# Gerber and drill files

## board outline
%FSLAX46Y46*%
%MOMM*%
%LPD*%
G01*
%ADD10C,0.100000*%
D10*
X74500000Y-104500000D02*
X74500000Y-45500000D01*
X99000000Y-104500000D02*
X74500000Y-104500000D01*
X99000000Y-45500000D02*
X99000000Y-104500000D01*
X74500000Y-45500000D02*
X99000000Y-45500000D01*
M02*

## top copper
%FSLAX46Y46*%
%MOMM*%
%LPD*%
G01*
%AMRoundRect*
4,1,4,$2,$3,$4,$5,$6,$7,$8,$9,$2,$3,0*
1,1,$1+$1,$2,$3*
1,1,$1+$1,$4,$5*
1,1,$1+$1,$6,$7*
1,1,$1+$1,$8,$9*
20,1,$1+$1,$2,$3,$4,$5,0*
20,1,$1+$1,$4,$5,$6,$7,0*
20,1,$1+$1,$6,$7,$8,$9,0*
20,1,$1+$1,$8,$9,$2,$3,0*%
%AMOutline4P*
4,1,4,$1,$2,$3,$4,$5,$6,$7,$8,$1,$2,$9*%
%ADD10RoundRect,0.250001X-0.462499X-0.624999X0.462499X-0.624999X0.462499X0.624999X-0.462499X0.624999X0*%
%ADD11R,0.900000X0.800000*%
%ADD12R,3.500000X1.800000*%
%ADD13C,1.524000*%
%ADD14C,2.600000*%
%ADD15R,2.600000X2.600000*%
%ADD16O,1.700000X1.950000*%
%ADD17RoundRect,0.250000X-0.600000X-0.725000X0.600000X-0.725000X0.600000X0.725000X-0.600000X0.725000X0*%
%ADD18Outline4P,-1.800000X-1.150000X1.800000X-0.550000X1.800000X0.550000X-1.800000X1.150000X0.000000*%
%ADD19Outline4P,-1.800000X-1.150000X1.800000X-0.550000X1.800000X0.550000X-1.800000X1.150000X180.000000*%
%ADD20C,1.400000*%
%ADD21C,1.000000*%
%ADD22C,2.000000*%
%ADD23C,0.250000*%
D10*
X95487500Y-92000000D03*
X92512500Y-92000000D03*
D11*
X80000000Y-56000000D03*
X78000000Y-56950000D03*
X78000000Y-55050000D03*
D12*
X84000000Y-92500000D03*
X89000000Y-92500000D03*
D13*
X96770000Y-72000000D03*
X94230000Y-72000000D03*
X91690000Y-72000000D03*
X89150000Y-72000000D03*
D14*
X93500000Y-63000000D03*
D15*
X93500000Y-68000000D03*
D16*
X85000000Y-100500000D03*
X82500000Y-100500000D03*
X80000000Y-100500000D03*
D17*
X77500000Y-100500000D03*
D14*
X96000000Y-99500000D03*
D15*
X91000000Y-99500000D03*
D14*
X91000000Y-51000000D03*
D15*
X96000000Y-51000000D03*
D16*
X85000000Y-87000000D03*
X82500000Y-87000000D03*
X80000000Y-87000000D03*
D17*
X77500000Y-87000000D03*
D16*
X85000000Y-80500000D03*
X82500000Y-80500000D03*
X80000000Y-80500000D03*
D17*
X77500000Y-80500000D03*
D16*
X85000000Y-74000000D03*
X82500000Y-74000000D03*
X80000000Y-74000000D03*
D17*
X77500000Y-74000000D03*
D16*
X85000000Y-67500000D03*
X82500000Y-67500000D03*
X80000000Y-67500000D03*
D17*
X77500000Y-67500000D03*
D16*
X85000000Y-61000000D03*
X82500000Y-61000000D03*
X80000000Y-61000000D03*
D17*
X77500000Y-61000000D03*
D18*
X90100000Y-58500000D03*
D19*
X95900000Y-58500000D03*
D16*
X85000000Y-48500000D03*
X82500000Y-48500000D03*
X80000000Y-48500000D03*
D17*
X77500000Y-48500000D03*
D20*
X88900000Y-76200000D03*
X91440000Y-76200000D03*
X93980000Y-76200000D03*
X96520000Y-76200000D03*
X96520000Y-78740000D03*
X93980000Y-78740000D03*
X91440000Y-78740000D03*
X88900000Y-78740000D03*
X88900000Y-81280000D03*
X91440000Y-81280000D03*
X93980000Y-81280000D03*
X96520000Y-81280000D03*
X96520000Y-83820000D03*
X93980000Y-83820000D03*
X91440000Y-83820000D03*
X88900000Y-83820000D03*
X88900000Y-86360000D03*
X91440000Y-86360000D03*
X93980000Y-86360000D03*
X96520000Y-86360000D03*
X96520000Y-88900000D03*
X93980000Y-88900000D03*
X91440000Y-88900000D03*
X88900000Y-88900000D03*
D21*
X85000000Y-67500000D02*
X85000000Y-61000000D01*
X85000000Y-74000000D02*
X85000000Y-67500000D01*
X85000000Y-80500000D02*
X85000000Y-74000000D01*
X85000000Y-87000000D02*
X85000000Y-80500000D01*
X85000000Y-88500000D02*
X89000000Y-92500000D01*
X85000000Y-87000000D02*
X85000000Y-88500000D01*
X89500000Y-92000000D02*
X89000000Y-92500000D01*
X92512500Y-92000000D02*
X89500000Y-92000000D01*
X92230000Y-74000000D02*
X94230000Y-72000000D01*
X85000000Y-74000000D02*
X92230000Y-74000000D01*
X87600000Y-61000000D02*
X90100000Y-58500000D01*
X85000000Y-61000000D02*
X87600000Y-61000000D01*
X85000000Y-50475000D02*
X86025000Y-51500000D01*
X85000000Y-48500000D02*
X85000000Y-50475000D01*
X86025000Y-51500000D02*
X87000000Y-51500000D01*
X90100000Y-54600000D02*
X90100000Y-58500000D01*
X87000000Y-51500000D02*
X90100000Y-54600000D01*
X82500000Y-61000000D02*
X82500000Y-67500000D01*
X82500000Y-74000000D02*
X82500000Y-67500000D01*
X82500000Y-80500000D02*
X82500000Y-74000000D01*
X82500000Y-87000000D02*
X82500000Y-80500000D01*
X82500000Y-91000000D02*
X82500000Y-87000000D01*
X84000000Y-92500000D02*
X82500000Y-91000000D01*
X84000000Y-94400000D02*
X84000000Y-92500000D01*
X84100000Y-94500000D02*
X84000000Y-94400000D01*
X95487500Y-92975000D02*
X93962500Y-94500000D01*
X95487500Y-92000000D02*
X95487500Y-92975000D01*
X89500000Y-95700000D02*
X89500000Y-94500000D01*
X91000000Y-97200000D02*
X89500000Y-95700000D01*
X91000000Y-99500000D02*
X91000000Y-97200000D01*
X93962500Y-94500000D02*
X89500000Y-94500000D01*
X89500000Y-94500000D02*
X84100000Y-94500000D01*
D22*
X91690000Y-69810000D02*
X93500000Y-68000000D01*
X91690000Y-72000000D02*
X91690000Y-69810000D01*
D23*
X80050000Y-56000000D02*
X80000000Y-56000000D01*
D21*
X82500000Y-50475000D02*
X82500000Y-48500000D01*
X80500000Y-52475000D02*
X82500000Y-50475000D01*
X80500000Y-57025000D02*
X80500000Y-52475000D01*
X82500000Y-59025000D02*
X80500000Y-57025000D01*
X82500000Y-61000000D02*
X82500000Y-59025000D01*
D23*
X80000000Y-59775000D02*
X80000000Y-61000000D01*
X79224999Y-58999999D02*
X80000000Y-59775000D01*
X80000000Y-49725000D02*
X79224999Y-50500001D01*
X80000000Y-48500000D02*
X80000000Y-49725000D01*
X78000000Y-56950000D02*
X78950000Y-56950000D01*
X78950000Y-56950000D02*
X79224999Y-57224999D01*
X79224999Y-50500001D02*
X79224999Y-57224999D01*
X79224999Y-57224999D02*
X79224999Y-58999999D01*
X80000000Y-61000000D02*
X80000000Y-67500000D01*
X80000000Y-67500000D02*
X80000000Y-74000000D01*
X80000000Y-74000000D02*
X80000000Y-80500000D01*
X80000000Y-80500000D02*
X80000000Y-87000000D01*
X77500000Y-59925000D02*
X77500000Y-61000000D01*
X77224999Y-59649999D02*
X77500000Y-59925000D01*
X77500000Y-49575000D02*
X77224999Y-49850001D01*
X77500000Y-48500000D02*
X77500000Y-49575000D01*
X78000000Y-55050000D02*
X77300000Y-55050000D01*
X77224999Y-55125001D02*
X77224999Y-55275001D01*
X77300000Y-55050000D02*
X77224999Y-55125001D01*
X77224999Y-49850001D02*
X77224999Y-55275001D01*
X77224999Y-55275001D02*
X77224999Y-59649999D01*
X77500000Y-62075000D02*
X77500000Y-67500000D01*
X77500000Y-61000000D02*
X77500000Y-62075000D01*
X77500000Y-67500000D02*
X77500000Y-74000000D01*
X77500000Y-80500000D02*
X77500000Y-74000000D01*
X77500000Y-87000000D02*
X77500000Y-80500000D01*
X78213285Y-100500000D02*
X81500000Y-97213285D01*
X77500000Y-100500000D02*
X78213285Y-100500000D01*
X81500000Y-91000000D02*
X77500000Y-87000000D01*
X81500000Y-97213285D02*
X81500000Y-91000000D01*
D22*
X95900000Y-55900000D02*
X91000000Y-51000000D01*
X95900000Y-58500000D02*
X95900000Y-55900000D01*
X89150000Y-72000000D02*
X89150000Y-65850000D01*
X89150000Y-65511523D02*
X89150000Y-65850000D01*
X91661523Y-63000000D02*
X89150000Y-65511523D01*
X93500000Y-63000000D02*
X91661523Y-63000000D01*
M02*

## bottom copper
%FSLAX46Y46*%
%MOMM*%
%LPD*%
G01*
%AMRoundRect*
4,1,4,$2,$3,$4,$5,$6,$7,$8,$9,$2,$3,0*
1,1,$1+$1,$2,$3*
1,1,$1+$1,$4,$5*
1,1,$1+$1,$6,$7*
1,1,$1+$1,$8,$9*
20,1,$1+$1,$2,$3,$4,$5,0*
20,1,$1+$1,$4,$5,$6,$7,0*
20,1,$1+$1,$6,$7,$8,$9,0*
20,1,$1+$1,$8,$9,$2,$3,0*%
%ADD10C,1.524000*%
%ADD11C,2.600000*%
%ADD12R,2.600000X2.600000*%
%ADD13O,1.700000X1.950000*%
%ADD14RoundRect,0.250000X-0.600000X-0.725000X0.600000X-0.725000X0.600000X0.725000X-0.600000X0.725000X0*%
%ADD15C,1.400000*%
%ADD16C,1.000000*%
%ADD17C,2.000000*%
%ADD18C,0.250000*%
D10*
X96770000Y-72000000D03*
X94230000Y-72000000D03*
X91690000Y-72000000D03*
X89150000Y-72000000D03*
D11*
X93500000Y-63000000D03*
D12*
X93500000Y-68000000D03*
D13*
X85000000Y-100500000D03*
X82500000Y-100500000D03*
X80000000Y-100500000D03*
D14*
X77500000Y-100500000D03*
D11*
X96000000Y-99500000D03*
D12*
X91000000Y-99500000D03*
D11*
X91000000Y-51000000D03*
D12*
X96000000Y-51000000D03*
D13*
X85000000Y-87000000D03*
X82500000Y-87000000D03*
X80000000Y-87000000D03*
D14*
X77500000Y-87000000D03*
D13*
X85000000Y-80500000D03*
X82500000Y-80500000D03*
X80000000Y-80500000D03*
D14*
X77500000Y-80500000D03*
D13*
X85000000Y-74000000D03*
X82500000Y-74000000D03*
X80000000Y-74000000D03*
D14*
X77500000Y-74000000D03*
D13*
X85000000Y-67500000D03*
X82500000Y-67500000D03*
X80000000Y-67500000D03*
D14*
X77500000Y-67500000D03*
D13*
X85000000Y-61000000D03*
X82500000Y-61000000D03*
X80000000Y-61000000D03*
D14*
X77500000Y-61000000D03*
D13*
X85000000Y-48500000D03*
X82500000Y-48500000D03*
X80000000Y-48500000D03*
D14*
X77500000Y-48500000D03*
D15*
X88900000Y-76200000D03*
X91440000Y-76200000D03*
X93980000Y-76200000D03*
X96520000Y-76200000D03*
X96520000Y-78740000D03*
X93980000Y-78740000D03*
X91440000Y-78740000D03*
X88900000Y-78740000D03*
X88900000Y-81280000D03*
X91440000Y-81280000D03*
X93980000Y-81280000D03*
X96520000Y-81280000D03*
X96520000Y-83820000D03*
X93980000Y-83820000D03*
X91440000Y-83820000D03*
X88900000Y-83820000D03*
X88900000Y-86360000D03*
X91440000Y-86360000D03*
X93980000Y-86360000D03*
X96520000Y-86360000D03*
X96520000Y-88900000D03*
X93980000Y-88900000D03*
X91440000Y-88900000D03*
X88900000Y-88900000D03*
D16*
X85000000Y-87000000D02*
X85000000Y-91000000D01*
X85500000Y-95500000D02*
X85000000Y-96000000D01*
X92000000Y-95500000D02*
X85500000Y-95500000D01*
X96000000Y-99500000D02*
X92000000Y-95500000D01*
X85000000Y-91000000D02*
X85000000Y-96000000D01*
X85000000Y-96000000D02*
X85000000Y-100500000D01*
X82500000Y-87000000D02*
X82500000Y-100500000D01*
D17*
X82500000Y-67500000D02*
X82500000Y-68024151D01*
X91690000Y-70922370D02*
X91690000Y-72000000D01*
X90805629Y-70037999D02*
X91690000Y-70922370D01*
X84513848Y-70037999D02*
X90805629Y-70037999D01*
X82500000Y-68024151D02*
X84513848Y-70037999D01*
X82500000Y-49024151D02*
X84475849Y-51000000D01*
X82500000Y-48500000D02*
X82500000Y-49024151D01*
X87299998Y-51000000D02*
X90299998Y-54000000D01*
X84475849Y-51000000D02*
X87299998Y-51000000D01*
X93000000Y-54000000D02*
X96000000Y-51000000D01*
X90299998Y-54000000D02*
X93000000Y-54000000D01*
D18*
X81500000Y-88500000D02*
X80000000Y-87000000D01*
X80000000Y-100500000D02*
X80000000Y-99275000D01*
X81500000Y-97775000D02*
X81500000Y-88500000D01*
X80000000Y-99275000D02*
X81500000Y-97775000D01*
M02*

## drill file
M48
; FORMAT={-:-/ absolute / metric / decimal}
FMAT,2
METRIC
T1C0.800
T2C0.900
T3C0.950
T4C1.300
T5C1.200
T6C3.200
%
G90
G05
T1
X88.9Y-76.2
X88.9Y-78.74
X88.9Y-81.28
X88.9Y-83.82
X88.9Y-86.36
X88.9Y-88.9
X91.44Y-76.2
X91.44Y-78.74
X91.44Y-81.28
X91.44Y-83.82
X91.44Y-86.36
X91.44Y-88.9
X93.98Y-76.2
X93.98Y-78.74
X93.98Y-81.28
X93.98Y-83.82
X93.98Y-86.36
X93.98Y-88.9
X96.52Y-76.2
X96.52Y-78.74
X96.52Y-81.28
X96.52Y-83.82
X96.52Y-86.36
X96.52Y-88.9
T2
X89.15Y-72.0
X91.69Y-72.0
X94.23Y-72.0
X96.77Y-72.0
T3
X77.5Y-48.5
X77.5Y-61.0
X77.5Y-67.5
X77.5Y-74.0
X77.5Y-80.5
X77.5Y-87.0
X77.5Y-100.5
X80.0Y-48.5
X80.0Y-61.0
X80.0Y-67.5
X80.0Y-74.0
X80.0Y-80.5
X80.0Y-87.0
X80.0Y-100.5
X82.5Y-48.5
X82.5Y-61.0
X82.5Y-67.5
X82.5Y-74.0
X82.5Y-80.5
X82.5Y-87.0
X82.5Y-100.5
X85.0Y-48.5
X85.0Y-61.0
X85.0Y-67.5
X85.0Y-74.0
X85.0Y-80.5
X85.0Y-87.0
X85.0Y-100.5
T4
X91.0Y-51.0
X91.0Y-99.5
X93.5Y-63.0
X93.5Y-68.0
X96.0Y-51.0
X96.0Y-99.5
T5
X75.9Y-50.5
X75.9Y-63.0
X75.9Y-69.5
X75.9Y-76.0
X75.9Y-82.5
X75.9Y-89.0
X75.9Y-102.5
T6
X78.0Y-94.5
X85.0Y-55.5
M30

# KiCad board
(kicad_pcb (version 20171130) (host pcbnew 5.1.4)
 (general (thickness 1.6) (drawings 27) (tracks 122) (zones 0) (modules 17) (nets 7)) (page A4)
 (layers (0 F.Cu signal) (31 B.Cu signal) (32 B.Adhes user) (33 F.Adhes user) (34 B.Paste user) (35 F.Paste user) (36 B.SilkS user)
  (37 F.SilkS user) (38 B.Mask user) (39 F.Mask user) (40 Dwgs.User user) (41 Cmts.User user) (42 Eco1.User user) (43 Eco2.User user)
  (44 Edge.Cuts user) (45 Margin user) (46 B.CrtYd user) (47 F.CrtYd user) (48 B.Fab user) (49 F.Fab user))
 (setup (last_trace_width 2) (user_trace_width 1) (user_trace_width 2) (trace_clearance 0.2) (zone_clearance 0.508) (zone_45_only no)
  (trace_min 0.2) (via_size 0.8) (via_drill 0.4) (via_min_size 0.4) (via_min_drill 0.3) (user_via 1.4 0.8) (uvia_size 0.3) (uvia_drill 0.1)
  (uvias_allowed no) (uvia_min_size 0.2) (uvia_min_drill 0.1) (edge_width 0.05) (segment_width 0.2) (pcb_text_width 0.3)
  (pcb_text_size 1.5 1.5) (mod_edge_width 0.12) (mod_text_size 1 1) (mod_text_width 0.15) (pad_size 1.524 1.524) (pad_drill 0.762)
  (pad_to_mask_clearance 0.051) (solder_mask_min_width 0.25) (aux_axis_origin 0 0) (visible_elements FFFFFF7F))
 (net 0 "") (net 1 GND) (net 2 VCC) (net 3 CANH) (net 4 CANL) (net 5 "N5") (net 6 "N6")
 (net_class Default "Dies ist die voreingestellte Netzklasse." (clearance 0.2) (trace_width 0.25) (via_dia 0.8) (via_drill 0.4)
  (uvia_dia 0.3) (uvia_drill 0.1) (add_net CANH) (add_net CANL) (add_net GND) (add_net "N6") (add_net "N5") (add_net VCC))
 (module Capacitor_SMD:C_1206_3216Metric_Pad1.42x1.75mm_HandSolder (layer F.Cu) (at 94 92)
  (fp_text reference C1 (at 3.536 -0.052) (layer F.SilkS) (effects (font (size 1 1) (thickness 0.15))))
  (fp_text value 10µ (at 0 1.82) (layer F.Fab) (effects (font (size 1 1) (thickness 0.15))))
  (pad 2 smd roundrect (at 1.4875 0) (size 1.425 1.75) (layers F.Cu F.Paste F.Mask) (roundrect_rratio 0.175439) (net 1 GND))
  (pad 1 smd roundrect (at -1.4875 0) (size 1.425 1.75) (layers F.Cu F.Paste F.Mask) (roundrect_rratio 0.175439) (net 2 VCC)))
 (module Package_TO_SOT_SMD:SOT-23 (layer F.Cu) (at 79 56)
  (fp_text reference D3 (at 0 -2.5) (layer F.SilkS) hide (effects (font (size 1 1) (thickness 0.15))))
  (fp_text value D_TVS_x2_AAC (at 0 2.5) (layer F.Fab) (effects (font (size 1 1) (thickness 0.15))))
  (pad 3 smd rect (at 1 0) (size 0.9 0.8) (layers F.Cu F.Paste F.Mask) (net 1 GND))
  (pad 2 smd rect (at -1 0.95) (size 0.9 0.8) (layers F.Cu F.Paste F.Mask) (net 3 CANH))
  (pad 1 smd rect (at -1 -0.95) (size 0.9 0.8) (layers F.Cu F.Paste F.Mask) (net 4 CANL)))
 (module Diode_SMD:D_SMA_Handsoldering (layer F.Cu) (at 86.5 92.5 180)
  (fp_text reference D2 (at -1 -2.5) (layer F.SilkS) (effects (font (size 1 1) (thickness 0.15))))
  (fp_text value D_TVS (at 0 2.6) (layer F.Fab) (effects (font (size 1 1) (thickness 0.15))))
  (pad 2 smd rect (at 2.5 0 180) (size 3.5 1.8) (layers F.Cu F.Paste F.Mask) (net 1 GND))
  (pad 1 smd rect (at -2.5 0 180) (size 3.5 1.8) (layers F.Cu F.Paste F.Mask) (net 2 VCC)))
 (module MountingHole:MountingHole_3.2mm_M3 (layer F.Cu) (at 78 94.5)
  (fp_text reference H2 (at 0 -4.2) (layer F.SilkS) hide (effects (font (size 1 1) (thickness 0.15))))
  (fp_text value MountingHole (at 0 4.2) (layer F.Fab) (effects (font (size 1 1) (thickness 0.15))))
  (pad 1 np_thru_hole circle (at 0 0) (size 3.2 3.2) (drill 3.2) (layers *.Cu *.Mask)))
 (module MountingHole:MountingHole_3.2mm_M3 (layer F.Cu) (at 85 55.5)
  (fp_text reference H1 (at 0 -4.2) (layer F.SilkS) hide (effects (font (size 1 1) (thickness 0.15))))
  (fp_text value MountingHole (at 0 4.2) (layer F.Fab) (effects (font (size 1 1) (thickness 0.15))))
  (pad 1 np_thru_hole circle (at 0 0) (size 3.2 3.2) (drill 3.2) (layers *.Cu *.Mask)))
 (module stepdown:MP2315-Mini (layer F.Cu) (at 93 81)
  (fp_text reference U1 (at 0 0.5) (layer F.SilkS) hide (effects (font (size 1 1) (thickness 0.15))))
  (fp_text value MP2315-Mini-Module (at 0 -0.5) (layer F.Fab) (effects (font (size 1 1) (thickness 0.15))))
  (pad 4 thru_hole circle (at 3.77 -9) (size 1.524 1.524) (drill 0.9) (layers *.Cu *.Mask))
  (pad 3 thru_hole circle (at 1.23 -9) (size 1.524 1.524) (drill 0.9) (layers *.Cu *.Mask) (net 2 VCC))
  (pad 2 thru_hole circle (at -1.31 -9) (size 1.524 1.524) (drill 0.9) (layers *.Cu *.Mask) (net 1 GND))
  (pad 1 thru_hole circle (at -3.85 -9) (size 1.524 1.524) (drill 0.9) (layers *.Cu *.Mask) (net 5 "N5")))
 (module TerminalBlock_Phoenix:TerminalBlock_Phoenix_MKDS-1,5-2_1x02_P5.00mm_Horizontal (layer F.Cu) (at 93.5 68 90)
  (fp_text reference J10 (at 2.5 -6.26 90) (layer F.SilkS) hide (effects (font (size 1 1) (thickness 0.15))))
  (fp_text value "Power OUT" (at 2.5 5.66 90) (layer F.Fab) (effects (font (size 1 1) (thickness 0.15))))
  (pad 2 thru_hole circle (at 5 0 90) (size 2.6 2.6) (drill 1.3) (layers *.Cu *.Mask) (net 5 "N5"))
  (pad 1 thru_hole rect (at 0 0 90) (size 2.6 2.6) (drill 1.3) (layers *.Cu *.Mask) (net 1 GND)))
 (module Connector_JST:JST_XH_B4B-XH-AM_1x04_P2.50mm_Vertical (layer F.Cu) (at 77.5 100.5)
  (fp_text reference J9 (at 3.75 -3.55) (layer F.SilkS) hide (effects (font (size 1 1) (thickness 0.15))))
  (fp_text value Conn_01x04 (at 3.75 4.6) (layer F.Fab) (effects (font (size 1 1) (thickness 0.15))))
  (pad "" np_thru_hole circle (at -1.6 2) (size 1.2 1.2) (drill 1.2) (layers *.Cu *.Mask))
  (pad 4 thru_hole oval (at 7.5 0) (size 1.7 1.95) (drill 0.95) (layers *.Cu *.Mask) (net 2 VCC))
  (pad 3 thru_hole oval (at 5 0) (size 1.7 1.95) (drill 0.95) (layers *.Cu *.Mask) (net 1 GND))
  (pad 2 thru_hole oval (at 2.5 0) (size 1.7 1.95) (drill 0.95) (layers *.Cu *.Mask) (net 3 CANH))
  (pad 1 thru_hole roundrect (at 0 0) (size 1.7 1.95) (drill 0.95) (layers *.Cu *.Mask) (roundrect_rratio 0.147059) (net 4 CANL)))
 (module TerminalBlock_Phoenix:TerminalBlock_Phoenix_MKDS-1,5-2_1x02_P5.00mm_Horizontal (layer F.Cu) (at 91 99.5)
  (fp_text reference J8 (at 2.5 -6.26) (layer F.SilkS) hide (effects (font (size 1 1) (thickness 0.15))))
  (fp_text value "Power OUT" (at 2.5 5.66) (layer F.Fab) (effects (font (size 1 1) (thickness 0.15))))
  (pad 2 thru_hole circle (at 5 0) (size 2.6 2.6) (drill 1.3) (layers *.Cu *.Mask) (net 2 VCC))
  (pad 1 thru_hole rect (at 0 0) (size 2.6 2.6) (drill 1.3) (layers *.Cu *.Mask) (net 1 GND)))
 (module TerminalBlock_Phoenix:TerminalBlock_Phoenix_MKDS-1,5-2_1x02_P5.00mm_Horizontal (layer F.Cu) (at 96 51 180)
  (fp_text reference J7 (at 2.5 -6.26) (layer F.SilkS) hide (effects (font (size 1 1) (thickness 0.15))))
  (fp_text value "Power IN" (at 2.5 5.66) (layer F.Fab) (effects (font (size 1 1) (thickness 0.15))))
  (pad 2 thru_hole circle (at 5 0 180) (size 2.6 2.6) (drill 1.3) (layers *.Cu *.Mask) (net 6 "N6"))
  (pad 1 thru_hole rect (at 0 0 180) (size 2.6 2.6) (drill 1.3) (layers *.Cu *.Mask) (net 1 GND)))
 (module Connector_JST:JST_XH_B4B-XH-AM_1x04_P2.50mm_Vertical (layer F.Cu) (at 77.5 87)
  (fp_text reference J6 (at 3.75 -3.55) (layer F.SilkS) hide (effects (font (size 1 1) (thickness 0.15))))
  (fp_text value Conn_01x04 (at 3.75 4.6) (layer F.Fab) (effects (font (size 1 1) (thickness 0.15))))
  (pad "" np_thru_hole circle (at -1.6 2) (size 1.2 1.2) (drill 1.2) (layers *.Cu *.Mask))
  (pad 4 thru_hole oval (at 7.5 0) (size 1.7 1.95) (drill 0.95) (layers *.Cu *.Mask) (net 2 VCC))
  (pad 3 thru_hole oval (at 5 0) (size 1.7 1.95) (drill 0.95) (layers *.Cu *.Mask) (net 1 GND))
  (pad 2 thru_hole oval (at 2.5 0) (size 1.7 1.95) (drill 0.95) (layers *.Cu *.Mask) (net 3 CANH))
  (pad 1 thru_hole roundrect (at 0 0) (size 1.7 1.95) (drill 0.95) (layers *.Cu *.Mask) (roundrect_rratio 0.147059) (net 4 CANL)))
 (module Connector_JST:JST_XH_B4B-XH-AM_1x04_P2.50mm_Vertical (layer F.Cu) (at 77.5 80.5)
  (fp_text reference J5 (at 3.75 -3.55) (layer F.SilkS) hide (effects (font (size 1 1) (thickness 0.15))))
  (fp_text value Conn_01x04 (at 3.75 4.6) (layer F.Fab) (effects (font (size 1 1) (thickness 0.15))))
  (pad "" np_thru_hole circle (at -1.6 2) (size 1.2 1.2) (drill 1.2) (layers *.Cu *.Mask))
  (pad 4 thru_hole oval (at 7.5 0) (size 1.7 1.95) (drill 0.95) (layers *.Cu *.Mask) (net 2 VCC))
  (pad 3 thru_hole oval (at 5 0) (size 1.7 1.95) (drill 0.95) (layers *.Cu *.Mask) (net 1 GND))
  (pad 2 thru_hole oval (at 2.5 0) (size 1.7 1.95) (drill 0.95) (layers *.Cu *.Mask) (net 3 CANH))
  (pad 1 thru_hole roundrect (at 0 0) (size 1.7 1.95) (drill 0.95) (layers *.Cu *.Mask) (roundrect_rratio 0.147059) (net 4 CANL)))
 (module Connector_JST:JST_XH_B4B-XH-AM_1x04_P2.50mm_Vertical (layer F.Cu) (at 77.5 74)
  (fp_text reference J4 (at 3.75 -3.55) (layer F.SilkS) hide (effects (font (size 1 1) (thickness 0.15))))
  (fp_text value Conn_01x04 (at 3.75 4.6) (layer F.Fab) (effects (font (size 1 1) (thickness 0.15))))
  (pad "" np_thru_hole circle (at -1.6 2) (size 1.2 1.2) (drill 1.2) (layers *.Cu *.Mask))
  (pad 4 thru_hole oval (at 7.5 0) (size 1.7 1.95) (drill 0.95) (layers *.Cu *.Mask) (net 2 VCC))
  (pad 3 thru_hole oval (at 5 0) (size 1.7 1.95) (drill 0.95) (layers *.Cu *.Mask) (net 1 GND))
  (pad 2 thru_hole oval (at 2.5 0) (size 1.7 1.95) (drill 0.95) (layers *.Cu *.Mask) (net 3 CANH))
  (pad 1 thru_hole roundrect (at 0 0) (size 1.7 1.95) (drill 0.95) (layers *.Cu *.Mask) (roundrect_rratio 0.147059) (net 4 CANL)))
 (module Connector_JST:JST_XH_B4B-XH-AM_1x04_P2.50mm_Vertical (layer F.Cu) (at 77.5 67.5)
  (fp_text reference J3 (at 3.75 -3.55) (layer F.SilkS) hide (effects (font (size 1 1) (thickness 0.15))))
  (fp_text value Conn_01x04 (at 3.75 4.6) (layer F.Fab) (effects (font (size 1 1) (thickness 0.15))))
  (pad "" np_thru_hole circle (at -1.6 2) (size 1.2 1.2) (drill 1.2) (layers *.Cu *.Mask))
  (pad 4 thru_hole oval (at 7.5 0) (size 1.7 1.95) (drill 0.95) (layers *.Cu *.Mask) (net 2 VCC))
  (pad 3 thru_hole oval (at 5 0) (size 1.7 1.95) (drill 0.95) (layers *.Cu *.Mask) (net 1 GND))
  (pad 2 thru_hole oval (at 2.5 0) (size 1.7 1.95) (drill 0.95) (layers *.Cu *.Mask) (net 3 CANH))
  (pad 1 thru_hole roundrect (at 0 0) (size 1.7 1.95) (drill 0.95) (layers *.Cu *.Mask) (roundrect_rratio 0.147059) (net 4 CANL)))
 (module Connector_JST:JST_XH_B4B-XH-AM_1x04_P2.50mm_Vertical (layer F.Cu) (at 77.5 61)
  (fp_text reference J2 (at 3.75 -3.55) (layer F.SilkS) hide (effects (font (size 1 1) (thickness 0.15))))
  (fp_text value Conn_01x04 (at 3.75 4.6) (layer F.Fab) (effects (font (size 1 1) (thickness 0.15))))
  (pad "" np_thru_hole circle (at -1.6 2) (size 1.2 1.2) (drill 1.2) (layers *.Cu *.Mask))
  (pad 4 thru_hole oval (at 7.5 0) (size 1.7 1.95) (drill 0.95) (layers *.Cu *.Mask) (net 2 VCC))
  (pad 3 thru_hole oval (at 5 0) (size 1.7 1.95) (drill 0.95) (layers *.Cu *.Mask) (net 1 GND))
  (pad 2 thru_hole oval (at 2.5 0) (size 1.7 1.95) (drill 0.95) (layers *.Cu *.Mask) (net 3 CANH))
  (pad 1 thru_hole roundrect (at 0 0) (size 1.7 1.95) (drill 0.95) (layers *.Cu *.Mask) (roundrect_rratio 0.147059) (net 4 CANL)))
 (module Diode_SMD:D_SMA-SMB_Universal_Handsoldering (layer F.Cu) (at 93 58.5 180)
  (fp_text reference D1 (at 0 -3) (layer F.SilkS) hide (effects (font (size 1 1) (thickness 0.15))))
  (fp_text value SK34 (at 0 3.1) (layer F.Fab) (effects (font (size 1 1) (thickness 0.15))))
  (pad 2 smd trapezoid (at 2.9 0) (size 3.6 1.7) (rect_delta 0.6 0) (layers F.Cu F.Paste F.Mask) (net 2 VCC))
  (pad 1 smd trapezoid (at -2.9 0 180) (size 3.6 1.7) (rect_delta 0.6 0) (layers F.Cu F.Paste F.Mask) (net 6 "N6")))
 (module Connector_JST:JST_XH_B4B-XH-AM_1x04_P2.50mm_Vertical (layer F.Cu) (at 77.5 48.5)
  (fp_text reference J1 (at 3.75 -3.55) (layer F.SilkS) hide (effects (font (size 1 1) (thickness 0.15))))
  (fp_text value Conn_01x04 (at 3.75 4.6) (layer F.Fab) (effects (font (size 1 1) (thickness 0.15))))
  (pad "" np_thru_hole circle (at -1.6 2) (size 1.2 1.2) (drill 1.2) (layers *.Cu *.Mask))
  (pad 4 thru_hole oval (at 7.5 0) (size 1.7 1.95) (drill 0.95) (layers *.Cu *.Mask) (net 2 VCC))
  (pad 3 thru_hole oval (at 5 0) (size 1.7 1.95) (drill 0.95) (layers *.Cu *.Mask) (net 1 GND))
  (pad 2 thru_hole oval (at 2.5 0) (size 1.7 1.95) (drill 0.95) (layers *.Cu *.Mask) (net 3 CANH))
  (pad 1 thru_hole roundrect (at 0 0) (size 1.7 1.95) (drill 0.95) (layers *.Cu *.Mask) (roundrect_rratio 0.147059) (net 4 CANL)))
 (gr_line (start 74.5 104.5) (end 74.5 45.5) (layer Edge.Cuts) (width 0.1))
 (gr_line (start 99 104.5) (end 74.5 104.5) (layer Edge.Cuts) (width 0.1))
 (gr_line (start 99 45.5) (end 99 104.5) (layer Edge.Cuts) (width 0.1))
 (gr_line (start 74.5 45.5) (end 99 45.5) (layer Edge.Cuts) (width 0.1))
 (via (at 88.9 76.2) (size 1.4) (drill 0.8) (layers F.Cu B.Cu) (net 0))
 (via (at 91.44 76.2) (size 1.4) (drill 0.8) (layers F.Cu B.Cu) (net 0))
 (via (at 93.98 76.2) (size 1.4) (drill 0.8) (layers F.Cu B.Cu) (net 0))
 (via (at 96.52 76.2) (size 1.4) (drill 0.8) (layers F.Cu B.Cu) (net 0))
 (via (at 96.52 78.74) (size 1.4) (drill 0.8) (layers F.Cu B.Cu) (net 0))
 (via (at 93.98 78.74) (size 1.4) (drill 0.8) (layers F.Cu B.Cu) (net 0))
 (via (at 91.44 78.74) (size 1.4) (drill 0.8) (layers F.Cu B.Cu) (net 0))
 (via (at 88.9 78.74) (size 1.4) (drill 0.8) (layers F.Cu B.Cu) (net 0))
 (via (at 88.9 81.28) (size 1.4) (drill 0.8) (layers F.Cu B.Cu) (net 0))
 (via (at 91.44 81.28) (size 1.4) (drill 0.8) (layers F.Cu B.Cu) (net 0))
 (via (at 93.98 81.28) (size 1.4) (drill 0.8) (layers F.Cu B.Cu) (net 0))
 (via (at 96.52 81.28) (size 1.4) (drill 0.8) (layers F.Cu B.Cu) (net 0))
 (via (at 96.52 83.82) (size 1.4) (drill 0.8) (layers F.Cu B.Cu) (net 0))
 (via (at 93.98 83.82) (size 1.4) (drill 0.8) (layers F.Cu B.Cu) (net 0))
 (via (at 91.44 83.82) (size 1.4) (drill 0.8) (layers F.Cu B.Cu) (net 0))
 (via (at 88.9 83.82) (size 1.4) (drill 0.8) (layers F.Cu B.Cu) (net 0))
 (via (at 88.9 86.36) (size 1.4) (drill 0.8) (layers F.Cu B.Cu) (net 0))
 (via (at 91.44 86.36) (size 1.4) (drill 0.8) (layers F.Cu B.Cu) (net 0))
 (via (at 93.98 86.36) (size 1.4) (drill 0.8) (layers F.Cu B.Cu) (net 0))
 (via (at 96.52 86.36) (size 1.4) (drill 0.8) (layers F.Cu B.Cu) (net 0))
 (via (at 96.52 88.9) (size 1.4) (drill 0.8) (layers F.Cu B.Cu) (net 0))
 (via (at 93.98 88.9) (size 1.4) (drill 0.8) (layers F.Cu B.Cu) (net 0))
 (via (at 91.44 88.9) (size 1.4) (drill 0.8) (layers F.Cu B.Cu) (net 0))
 (via (at 88.9 88.9) (size 1.4) (drill 0.8) (layers F.Cu B.Cu) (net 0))
 (segment (start 85 67.5) (end 85 61) (width 1) (layer F.Cu) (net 2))
 (segment (start 85 74) (end 85 67.5) (width 1) (layer F.Cu) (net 2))
 (segment (start 85 80.5) (end 85 74) (width 1) (layer F.Cu) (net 2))
 (segment (start 85 87) (end 85 80.5) (width 1) (layer F.Cu) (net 2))
 (segment (start 85 88.5) (end 89 92.5) (width 1) (layer F.Cu) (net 2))
 (segment (start 85 87) (end 85 88.5) (width 1) (layer F.Cu) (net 2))
 (segment (start 89.5 92) (end 89 92.5) (width 1) (layer F.Cu) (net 2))
 (segment (start 92.5125 92) (end 89.5 92) (width 1) (layer F.Cu) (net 2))
 (segment (start 85 87) (end 85 91) (width 1) (layer B.Cu) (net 2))
 (segment (start 85.5 95.5) (end 85 96) (width 1) (layer B.Cu) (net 2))
 (segment (start 92 95.5) (end 85.5 95.5) (width 1) (layer B.Cu) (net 2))
 (segment (start 96 99.5) (end 92 95.5) (width 1) (layer B.Cu) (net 2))
 (segment (start 85 91) (end 85 96) (width 1) (layer B.Cu) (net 2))
 (segment (start 85 96) (end 85 100.5) (width 1) (layer B.Cu) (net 2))
 (segment (start 92.23 74) (end 94.23 72) (width 1) (layer F.Cu) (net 2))
 (segment (start 85 74) (end 92.23 74) (width 1) (layer F.Cu) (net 2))
 (segment (start 87.6 61) (end 90.1 58.5) (width 1) (layer F.Cu) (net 2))
 (segment (start 85 61) (end 87.6 61) (width 1) (layer F.Cu) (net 2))
 (segment (start 85 50.475) (end 86.025 51.5) (width 1) (layer F.Cu) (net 2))
 (segment (start 85 48.5) (end 85 50.475) (width 1) (layer F.Cu) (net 2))
 (segment (start 86.025 51.5) (end 87 51.5) (width 1) (layer F.Cu) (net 2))
 (segment (start 90.1 54.6) (end 90.1 58.5) (width 1) (layer F.Cu) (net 2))
 (segment (start 87 51.5) (end 90.1 54.6) (width 1) (layer F.Cu) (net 2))
 (segment (start 82.5 61) (end 82.5 67.5) (width 1) (layer F.Cu) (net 1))
 (segment (start 82.5 74) (end 82.5 67.5) (width 1) (layer F.Cu) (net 1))
 (segment (start 82.5 80.5) (end 82.5 74) (width 1) (layer F.Cu) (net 1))
 (segment (start 82.5 87) (end 82.5 80.5) (width 1) (layer F.Cu) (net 1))
 (segment (start 82.5 91) (end 82.5 87) (width 1) (layer F.Cu) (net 1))
 (segment (start 84 92.5) (end 82.5 91) (width 1) (layer F.Cu) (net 1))
 (segment (start 84 94.4) (end 84 92.5) (width 1) (layer F.Cu) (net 1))
 (segment (start 84.1 94.5) (end 84 94.4) (width 1) (layer F.Cu) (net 1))
 (segment (start 95.4875 92.975) (end 93.9625 94.5) (width 1) (layer F.Cu) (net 1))
 (segment (start 95.4875 92) (end 95.4875 92.975) (width 1) (layer F.Cu) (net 1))
 (segment (start 82.5 87) (end 82.5 100.5) (width 1) (layer B.Cu) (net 1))
 (segment (start 89.5 95.7) (end 89.5 94.5) (width 1) (layer F.Cu) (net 1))
 (segment (start 91 97.2) (end 89.5 95.7) (width 1) (layer F.Cu) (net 1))
 (segment (start 91 99.5) (end 91 97.2) (width 1) (layer F.Cu) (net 1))
 (segment (start 93.9625 94.5) (end 89.5 94.5) (width 1) (layer F.Cu) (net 1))
 (segment (start 89.5 94.5) (end 84.1 94.5) (width 1) (layer F.Cu) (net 1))
 (segment (start 91.69 69.81) (end 93.5 68) (width 2) (layer F.Cu) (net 1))
 (segment (start 91.69 72) (end 91.69 69.81) (width 2) (layer F.Cu) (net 1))
 (segment (start 82.5 67.5) (end 82.5 68.024151) (width 2) (layer B.Cu) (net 1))
 (segment (start 91.69 70.92237) (end 91.69 72) (width 2) (layer B.Cu) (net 1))
 (segment (start 90.805629 70.037999) (end 91.69 70.92237) (width 2) (layer B.Cu) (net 1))
 (segment (start 84.513848 70.037999) (end 90.805629 70.037999) (width 2) (layer B.Cu) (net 1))
 (segment (start 82.5 68.024151) (end 84.513848 70.037999) (width 2) (layer B.Cu) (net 1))
 (segment (start 80.05 56) (end 80 56) (width 0.25) (layer F.Cu) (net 1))
 (segment (start 82.5 50.475) (end 82.5 48.5) (width 1) (layer F.Cu) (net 1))
 (segment (start 80.5 52.475) (end 82.5 50.475) (width 1) (layer F.Cu) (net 1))
 (segment (start 80.5 57.025) (end 80.5 52.475) (width 1) (layer F.Cu) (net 1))
 (segment (start 82.5 59.025) (end 80.5 57.025) (width 1) (layer F.Cu) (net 1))
 (segment (start 82.5 61) (end 82.5 59.025) (width 1) (layer F.Cu) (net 1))
 (segment (start 82.5 49.024151) (end 84.475849 51) (width 2) (layer B.Cu) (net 1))
 (segment (start 82.5 48.5) (end 82.5 49.024151) (width 2) (layer B.Cu) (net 1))
 (segment (start 87.299998 51) (end 90.299998 54) (width 2) (layer B.Cu) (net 1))
 (segment (start 84.475849 51) (end 87.299998 51) (width 2) (layer B.Cu) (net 1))
 (segment (start 93 54) (end 96 51) (width 2) (layer B.Cu) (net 1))
 (segment (start 90.299998 54) (end 93 54) (width 2) (layer B.Cu) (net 1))
 (segment (start 80 59.775) (end 80 61) (width 0.25) (layer F.Cu) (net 3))
 (segment (start 79.224999 58.999999) (end 80 59.775) (width 0.25) (layer F.Cu) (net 3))
 (segment (start 80 49.725) (end 79.224999 50.500001) (width 0.25) (layer F.Cu) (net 3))
 (segment (start 80 48.5) (end 80 49.725) (width 0.25) (layer F.Cu) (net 3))
 (segment (start 78 56.95) (end 78.95 56.95) (width 0.25) (layer F.Cu) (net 3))
 (segment (start 78.95 56.95) (end 79.224999 57.224999) (width 0.25) (layer F.Cu) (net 3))
 (segment (start 79.224999 50.500001) (end 79.224999 57.224999) (width 0.25) (layer F.Cu) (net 3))
 (segment (start 79.224999 57.224999) (end 79.224999 58.999999) (width 0.25) (layer F.Cu) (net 3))
 (segment (start 81.5 88.5) (end 80 87) (width 0.25) (layer B.Cu) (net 3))
 (segment (start 80 100.5) (end 80 99.275) (width 0.25) (layer B.Cu) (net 3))
 (segment (start 81.5 97.775) (end 81.5 88.5) (width 0.25) (layer B.Cu) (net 3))
 (segment (start 80 99.275) (end 81.5 97.775) (width 0.25) (layer B.Cu) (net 3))
 (segment (start 80 61) (end 80 67.5) (width 0.25) (layer F.Cu) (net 3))
 (segment (start 80 67.5) (end 80 74) (width 0.25) (layer F.Cu) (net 3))
 (segment (start 80 74) (end 80 80.5) (width 0.25) (layer F.Cu) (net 3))
 (segment (start 80 80.5) (end 80 87) (width 0.25) (layer F.Cu) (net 3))
 (segment (start 77.5 59.925) (end 77.5 61) (width 0.25) (layer F.Cu) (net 4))
 (segment (start 77.224999 59.649999) (end 77.5 59.925) (width 0.25) (layer F.Cu) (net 4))
 (segment (start 77.5 49.575) (end 77.224999 49.850001) (width 0.25) (layer F.Cu) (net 4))
 (segment (start 77.5 48.5) (end 77.5 49.575) (width 0.25) (layer F.Cu) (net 4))
 (segment (start 78 55.05) (end 77.3 55.05) (width 0.25) (layer F.Cu) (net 4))
 (segment (start 77.224999 55.125001) (end 77.224999 55.275001) (width 0.25) (layer F.Cu) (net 4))
 (segment (start 77.3 55.05) (end 77.224999 55.125001) (width 0.25) (layer F.Cu) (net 4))
 (segment (start 77.224999 49.850001) (end 77.224999 55.275001) (width 0.25) (layer F.Cu) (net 4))
 (segment (start 77.224999 55.275001) (end 77.224999 59.649999) (width 0.25) (layer F.Cu) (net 4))
 (segment (start 77.5 62.075) (end 77.5 67.5) (width 0.25) (layer F.Cu) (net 4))
 (segment (start 77.5 61) (end 77.5 62.075) (width 0.25) (layer F.Cu) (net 4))
 (segment (start 77.5 67.5) (end 77.5 74) (width 0.25) (layer F.Cu) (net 4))
 (segment (start 77.5 80.5) (end 77.5 74) (width 0.25) (layer F.Cu) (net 4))
 (segment (start 77.5 87) (end 77.5 80.5) (width 0.25) (layer F.Cu) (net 4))
 (segment (start 78.213285 100.5) (end 81.5 97.213285) (width 0.25) (layer F.Cu) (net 4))
 (segment (start 77.5 100.5) (end 78.213285 100.5) (width 0.25) (layer F.Cu) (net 4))
 (segment (start 81.5 91) (end 77.5 87) (width 0.25) (layer F.Cu) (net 4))
 (segment (start 81.5 97.213285) (end 81.5 91) (width 0.25) (layer F.Cu) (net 4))
 (segment (start 95.9 55.9) (end 91 51) (width 2) (layer F.Cu) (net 6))
 (segment (start 95.9 58.5) (end 95.9 55.9) (width 2) (layer F.Cu) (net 6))
 (segment (start 89.15 72) (end 89.15 65.85) (width 2) (layer F.Cu) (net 5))
 (segment (start 89.15 65.511523) (end 89.15 65.85) (width 2) (layer F.Cu) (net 5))
 (segment (start 91.661523 63) (end 89.15 65.511523) (width 2) (layer F.Cu) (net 5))
 (segment (start 93.5 63) (end 91.661523 63) (width 2) (layer F.Cu) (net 5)))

